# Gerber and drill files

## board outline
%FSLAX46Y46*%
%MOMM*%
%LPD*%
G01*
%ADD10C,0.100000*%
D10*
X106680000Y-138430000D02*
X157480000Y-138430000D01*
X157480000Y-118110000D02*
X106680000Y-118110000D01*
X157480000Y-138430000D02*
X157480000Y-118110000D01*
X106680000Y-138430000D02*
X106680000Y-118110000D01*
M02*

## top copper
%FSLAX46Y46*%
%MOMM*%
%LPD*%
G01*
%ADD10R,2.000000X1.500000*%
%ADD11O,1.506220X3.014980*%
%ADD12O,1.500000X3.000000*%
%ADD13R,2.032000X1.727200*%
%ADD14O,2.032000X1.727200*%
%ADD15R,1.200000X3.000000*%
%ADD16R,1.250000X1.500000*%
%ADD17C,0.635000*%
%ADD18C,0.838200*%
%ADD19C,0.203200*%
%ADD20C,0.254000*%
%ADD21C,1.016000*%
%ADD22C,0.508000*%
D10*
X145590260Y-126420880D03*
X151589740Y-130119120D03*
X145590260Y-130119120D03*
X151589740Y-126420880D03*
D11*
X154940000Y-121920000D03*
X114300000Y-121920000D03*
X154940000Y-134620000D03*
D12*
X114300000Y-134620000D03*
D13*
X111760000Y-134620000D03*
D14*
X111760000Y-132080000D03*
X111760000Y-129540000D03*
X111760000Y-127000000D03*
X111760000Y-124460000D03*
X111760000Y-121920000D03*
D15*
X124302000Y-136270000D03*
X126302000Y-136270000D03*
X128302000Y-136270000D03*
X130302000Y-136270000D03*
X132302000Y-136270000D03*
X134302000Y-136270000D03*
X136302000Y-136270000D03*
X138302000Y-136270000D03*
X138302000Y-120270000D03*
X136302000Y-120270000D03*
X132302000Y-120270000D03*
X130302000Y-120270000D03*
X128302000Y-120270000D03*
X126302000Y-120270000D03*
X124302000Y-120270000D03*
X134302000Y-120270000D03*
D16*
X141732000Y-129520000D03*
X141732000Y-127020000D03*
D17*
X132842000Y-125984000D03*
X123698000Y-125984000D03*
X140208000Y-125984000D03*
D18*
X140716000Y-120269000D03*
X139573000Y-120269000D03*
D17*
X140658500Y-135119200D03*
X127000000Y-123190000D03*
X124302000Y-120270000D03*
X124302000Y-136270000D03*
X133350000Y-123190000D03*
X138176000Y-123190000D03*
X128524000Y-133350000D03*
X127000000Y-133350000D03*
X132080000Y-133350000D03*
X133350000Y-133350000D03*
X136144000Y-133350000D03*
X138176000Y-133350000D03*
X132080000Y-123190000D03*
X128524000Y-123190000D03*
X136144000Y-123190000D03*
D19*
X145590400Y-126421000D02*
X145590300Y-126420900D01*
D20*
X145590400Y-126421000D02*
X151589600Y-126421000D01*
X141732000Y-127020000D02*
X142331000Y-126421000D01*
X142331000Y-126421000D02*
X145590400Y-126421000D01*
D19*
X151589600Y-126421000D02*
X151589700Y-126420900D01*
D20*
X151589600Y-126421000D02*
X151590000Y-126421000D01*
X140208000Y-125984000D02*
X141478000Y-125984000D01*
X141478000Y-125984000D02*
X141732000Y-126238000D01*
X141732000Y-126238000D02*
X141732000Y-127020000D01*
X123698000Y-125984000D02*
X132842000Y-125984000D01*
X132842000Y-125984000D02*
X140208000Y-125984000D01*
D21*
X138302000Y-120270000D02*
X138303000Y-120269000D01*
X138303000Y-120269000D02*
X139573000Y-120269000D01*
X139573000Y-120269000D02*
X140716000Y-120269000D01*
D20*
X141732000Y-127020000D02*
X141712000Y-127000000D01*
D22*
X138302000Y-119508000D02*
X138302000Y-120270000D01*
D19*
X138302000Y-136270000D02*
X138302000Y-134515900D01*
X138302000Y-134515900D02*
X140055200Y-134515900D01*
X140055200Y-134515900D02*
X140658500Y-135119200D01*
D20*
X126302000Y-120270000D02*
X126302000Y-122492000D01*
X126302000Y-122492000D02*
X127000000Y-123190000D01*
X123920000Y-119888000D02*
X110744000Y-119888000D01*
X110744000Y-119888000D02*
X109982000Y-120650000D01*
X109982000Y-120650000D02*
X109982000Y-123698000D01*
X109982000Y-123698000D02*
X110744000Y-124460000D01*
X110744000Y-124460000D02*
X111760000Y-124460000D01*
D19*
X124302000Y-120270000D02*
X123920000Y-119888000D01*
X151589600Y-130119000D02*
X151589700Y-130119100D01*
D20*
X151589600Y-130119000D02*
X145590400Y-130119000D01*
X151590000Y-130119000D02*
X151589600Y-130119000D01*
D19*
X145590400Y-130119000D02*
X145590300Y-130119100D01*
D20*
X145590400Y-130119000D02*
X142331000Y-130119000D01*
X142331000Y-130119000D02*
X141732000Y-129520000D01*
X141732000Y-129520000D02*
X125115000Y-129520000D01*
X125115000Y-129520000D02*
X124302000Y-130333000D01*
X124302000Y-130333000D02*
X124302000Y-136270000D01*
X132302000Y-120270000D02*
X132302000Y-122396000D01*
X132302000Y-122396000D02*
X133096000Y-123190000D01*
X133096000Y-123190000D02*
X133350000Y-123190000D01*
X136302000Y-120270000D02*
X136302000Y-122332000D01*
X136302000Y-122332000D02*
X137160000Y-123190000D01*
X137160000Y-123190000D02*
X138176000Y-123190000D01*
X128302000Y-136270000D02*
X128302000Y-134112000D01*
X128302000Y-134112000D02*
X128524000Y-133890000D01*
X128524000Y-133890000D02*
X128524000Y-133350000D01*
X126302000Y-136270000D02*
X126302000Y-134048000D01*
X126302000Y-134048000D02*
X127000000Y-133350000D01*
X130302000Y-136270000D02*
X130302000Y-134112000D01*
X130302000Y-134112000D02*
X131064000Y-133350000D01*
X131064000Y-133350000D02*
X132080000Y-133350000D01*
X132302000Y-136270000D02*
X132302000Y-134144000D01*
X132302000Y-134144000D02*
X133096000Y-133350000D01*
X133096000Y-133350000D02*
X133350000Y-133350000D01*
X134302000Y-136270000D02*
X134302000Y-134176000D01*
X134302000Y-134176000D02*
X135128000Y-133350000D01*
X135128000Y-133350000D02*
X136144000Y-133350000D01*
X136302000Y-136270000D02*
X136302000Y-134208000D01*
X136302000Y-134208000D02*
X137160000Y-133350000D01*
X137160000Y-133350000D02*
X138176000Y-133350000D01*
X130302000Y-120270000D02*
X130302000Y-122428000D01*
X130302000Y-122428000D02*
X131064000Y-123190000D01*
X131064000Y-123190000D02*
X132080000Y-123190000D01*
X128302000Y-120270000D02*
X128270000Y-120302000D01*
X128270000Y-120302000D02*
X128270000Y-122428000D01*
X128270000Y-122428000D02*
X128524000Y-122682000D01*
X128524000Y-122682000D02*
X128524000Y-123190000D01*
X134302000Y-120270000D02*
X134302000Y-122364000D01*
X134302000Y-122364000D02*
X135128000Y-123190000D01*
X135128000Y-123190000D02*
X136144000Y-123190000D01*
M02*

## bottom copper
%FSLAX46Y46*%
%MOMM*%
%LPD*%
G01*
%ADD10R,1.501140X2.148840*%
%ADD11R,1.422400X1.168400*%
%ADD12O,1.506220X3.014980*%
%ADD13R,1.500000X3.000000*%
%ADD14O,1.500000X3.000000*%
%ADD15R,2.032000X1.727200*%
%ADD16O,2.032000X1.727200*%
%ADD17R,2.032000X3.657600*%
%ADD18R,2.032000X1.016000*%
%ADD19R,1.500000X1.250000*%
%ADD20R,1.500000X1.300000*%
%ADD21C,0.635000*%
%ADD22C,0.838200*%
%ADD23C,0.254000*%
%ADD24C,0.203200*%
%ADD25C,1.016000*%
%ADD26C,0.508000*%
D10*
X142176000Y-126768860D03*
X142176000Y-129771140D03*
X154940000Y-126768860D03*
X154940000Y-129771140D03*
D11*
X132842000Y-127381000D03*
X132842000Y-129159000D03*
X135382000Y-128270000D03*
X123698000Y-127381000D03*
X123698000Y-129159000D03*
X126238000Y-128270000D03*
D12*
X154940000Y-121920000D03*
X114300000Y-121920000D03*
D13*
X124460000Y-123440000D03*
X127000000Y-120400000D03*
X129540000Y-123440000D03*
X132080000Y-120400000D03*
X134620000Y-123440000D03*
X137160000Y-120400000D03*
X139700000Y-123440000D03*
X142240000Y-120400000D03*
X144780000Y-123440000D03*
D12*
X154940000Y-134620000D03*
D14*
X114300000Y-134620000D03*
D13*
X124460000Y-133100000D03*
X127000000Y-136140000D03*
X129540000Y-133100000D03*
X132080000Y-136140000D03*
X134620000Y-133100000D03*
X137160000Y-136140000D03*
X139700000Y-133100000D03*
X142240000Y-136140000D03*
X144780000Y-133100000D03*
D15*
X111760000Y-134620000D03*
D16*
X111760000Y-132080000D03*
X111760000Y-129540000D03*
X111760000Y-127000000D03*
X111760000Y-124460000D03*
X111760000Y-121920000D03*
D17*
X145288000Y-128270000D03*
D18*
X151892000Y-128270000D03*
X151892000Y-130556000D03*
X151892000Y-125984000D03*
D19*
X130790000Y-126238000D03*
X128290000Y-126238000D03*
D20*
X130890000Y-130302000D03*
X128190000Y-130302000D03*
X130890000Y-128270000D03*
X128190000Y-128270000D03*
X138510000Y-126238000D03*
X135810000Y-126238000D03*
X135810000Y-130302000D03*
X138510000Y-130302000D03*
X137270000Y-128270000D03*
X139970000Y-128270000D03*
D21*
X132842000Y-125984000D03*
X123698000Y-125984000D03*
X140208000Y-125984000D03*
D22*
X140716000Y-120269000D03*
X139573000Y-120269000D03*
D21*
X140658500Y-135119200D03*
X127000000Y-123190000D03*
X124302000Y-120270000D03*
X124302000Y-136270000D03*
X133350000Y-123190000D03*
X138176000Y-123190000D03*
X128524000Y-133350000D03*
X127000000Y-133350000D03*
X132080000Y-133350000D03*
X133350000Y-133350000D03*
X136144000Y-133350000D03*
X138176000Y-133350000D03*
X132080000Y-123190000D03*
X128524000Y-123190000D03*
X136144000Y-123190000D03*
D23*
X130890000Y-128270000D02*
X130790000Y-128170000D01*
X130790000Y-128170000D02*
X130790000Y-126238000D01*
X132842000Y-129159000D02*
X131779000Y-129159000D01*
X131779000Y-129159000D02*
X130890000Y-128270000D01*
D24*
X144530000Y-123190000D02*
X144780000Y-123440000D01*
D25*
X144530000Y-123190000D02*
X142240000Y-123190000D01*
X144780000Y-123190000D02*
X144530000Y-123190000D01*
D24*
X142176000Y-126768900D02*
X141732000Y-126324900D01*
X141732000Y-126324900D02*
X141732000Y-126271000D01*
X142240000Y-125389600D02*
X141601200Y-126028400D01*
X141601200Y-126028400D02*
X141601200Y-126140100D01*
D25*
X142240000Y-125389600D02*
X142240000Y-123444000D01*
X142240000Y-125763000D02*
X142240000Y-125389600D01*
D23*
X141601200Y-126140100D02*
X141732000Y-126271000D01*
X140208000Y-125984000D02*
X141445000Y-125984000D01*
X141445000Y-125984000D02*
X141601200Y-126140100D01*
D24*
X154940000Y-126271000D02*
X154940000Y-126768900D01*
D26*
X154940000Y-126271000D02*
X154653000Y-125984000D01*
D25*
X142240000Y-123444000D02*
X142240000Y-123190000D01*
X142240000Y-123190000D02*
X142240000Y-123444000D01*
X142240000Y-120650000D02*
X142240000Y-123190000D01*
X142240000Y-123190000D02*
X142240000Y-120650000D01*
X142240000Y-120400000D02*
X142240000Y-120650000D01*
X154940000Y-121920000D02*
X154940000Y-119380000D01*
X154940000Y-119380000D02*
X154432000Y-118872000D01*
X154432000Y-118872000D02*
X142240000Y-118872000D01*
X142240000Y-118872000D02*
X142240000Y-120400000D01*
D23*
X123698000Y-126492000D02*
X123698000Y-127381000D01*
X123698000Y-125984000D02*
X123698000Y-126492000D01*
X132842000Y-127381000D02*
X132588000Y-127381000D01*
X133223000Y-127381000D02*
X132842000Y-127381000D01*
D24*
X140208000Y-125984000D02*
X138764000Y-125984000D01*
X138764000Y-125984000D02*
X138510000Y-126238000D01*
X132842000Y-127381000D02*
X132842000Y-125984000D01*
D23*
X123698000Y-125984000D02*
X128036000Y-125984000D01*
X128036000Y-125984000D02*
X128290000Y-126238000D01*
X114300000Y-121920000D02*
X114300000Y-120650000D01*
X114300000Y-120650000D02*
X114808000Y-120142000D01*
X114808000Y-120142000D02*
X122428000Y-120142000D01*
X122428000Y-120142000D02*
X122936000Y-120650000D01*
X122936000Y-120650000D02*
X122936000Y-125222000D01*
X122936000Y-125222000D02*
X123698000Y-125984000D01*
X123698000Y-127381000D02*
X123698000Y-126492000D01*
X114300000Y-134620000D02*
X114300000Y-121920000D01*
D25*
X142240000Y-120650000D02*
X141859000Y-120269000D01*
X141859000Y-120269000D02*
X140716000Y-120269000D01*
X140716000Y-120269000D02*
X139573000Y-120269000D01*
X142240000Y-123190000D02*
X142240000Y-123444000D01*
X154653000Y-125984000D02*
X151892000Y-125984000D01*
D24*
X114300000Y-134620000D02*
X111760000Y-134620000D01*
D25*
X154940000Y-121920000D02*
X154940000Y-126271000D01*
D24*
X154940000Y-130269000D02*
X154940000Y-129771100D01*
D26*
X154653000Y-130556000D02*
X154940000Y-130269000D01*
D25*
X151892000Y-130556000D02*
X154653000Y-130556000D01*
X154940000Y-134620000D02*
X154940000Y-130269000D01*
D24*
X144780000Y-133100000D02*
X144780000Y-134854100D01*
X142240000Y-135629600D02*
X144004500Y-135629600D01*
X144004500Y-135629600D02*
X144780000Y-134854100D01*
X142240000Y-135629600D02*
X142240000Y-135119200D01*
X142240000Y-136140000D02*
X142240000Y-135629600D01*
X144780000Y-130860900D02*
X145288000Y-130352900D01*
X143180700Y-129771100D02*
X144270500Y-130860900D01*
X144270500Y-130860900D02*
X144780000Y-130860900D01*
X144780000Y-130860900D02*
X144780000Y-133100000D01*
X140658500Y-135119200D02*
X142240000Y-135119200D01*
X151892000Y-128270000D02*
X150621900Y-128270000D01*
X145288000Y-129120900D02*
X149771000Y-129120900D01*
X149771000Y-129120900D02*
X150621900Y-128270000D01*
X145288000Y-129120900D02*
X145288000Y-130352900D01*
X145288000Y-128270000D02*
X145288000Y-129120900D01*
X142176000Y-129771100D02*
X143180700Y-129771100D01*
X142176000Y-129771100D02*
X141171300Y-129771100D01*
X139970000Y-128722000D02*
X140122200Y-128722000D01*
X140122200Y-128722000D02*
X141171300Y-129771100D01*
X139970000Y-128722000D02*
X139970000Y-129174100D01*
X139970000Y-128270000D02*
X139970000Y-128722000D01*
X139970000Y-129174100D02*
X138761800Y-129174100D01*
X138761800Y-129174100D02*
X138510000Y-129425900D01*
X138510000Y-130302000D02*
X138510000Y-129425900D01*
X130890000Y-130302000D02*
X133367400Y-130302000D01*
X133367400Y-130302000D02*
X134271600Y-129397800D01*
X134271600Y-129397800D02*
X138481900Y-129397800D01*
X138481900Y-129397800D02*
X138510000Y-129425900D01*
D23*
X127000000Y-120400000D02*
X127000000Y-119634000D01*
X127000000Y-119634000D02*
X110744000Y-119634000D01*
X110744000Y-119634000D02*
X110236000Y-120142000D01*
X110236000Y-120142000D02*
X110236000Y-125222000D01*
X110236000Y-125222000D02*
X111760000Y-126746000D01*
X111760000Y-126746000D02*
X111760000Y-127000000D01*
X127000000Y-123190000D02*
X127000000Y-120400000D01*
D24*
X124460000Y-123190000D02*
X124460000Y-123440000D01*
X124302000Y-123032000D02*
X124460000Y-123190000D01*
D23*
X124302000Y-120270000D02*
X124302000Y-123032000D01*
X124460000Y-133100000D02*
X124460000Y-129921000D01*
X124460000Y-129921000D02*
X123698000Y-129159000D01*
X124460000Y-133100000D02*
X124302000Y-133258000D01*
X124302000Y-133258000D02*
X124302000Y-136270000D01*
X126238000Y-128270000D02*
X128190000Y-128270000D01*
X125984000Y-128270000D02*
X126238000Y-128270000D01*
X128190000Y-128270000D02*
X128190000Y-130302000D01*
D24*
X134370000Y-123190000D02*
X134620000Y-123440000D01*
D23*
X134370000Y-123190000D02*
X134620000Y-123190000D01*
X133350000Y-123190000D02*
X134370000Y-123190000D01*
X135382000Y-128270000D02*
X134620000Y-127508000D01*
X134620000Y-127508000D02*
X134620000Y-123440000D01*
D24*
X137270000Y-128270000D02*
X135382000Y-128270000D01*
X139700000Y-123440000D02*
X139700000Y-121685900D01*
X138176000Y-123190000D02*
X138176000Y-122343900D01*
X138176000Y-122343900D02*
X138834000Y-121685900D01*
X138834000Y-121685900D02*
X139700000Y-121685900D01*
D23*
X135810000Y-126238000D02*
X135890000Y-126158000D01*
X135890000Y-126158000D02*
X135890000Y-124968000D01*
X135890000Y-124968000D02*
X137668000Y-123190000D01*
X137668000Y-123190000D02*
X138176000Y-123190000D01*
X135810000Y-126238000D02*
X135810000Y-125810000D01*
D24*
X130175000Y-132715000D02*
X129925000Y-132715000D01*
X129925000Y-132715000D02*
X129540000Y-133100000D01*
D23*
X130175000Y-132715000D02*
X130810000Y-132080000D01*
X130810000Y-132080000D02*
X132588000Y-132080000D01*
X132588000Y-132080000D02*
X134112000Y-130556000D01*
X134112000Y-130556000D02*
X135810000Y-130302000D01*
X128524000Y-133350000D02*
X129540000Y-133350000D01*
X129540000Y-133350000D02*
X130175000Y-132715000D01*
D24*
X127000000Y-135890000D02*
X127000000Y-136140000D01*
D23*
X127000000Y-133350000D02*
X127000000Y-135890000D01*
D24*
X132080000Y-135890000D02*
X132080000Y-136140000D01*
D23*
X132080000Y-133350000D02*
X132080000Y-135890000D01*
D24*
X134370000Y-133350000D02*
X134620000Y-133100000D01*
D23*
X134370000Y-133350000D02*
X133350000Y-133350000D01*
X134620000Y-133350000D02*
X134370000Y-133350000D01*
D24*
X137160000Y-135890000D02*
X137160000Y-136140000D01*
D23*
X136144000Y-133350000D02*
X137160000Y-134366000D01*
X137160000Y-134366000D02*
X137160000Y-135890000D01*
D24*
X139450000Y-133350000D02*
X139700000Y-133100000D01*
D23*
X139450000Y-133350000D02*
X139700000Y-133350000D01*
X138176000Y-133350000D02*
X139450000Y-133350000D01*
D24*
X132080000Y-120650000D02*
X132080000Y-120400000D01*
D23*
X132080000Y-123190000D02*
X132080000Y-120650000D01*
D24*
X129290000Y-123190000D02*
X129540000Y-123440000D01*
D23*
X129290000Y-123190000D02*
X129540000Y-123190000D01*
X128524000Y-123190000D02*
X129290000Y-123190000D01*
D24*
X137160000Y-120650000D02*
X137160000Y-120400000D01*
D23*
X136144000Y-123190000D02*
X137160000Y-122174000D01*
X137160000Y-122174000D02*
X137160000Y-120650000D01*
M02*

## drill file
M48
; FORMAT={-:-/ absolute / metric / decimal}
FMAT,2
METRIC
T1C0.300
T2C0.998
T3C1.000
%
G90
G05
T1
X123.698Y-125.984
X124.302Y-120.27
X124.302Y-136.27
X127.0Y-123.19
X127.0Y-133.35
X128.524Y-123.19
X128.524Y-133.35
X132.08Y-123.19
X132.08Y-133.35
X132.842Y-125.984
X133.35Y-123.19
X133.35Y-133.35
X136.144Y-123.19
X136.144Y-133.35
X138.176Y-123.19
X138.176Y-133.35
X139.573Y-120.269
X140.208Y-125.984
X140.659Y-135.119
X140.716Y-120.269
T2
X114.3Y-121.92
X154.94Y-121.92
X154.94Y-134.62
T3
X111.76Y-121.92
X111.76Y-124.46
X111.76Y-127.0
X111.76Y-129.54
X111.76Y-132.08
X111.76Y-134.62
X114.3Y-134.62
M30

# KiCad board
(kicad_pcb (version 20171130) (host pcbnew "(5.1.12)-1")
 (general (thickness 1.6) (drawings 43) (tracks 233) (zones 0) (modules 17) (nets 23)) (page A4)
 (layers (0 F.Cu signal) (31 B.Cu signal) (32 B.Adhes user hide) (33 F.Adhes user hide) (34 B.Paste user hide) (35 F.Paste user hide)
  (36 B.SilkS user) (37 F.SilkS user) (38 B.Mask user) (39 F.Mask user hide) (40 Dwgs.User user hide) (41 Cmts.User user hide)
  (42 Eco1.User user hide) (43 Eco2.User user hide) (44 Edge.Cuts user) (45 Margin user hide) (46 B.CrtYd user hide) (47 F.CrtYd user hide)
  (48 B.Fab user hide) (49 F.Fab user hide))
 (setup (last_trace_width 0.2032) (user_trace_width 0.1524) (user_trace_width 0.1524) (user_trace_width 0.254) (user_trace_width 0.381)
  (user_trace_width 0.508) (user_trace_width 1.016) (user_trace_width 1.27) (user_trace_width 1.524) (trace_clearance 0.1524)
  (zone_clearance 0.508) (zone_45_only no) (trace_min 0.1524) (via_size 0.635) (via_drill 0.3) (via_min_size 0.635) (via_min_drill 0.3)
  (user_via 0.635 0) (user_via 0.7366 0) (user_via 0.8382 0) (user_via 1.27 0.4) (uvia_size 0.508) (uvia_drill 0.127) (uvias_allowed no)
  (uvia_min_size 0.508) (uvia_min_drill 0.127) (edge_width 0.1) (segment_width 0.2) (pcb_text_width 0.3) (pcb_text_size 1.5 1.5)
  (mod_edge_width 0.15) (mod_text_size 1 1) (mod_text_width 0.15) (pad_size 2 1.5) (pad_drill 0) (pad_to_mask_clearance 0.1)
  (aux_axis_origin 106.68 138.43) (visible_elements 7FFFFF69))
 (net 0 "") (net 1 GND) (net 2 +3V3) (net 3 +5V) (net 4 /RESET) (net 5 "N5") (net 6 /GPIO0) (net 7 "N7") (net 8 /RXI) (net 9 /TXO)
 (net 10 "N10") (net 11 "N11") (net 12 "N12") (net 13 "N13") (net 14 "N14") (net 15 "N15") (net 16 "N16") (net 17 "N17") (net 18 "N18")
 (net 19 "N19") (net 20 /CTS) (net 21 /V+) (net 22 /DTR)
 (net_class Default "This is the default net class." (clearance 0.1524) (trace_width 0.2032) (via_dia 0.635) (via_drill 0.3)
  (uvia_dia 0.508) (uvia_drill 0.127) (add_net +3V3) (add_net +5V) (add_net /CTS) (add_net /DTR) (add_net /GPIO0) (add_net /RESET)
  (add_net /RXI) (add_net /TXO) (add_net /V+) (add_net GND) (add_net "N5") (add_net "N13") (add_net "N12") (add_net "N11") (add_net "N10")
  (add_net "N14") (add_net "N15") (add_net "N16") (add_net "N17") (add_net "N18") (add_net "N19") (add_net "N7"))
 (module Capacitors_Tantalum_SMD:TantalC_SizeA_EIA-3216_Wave (layer B.Cu) (at 142.176 128.27 90)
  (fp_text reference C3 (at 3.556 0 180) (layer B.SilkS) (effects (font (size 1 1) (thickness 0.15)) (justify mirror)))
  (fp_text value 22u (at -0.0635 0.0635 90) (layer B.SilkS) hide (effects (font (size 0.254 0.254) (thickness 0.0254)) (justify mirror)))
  (pad 2 smd rect (at 1.50114 0 90) (size 2.14884 1.50114) (layers B.Cu B.Paste B.Mask) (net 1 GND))
  (pad 1 smd rect (at -1.50114 0 90) (size 2.14884 1.50114) (layers B.Cu B.Paste B.Mask) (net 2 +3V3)))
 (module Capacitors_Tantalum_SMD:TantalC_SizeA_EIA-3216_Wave (layer B.Cu) (at 154.94 128.27 90)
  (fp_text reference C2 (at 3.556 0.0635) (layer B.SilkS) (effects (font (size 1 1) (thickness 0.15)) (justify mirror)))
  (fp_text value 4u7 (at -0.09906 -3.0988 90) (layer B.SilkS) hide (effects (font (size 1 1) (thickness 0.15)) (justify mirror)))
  (pad 2 smd rect (at 1.50114 0 90) (size 2.14884 1.50114) (layers B.Cu B.Paste B.Mask) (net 1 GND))
  (pad 1 smd rect (at -1.50114 0 90) (size 2.14884 1.50114) (layers B.Cu B.Paste B.Mask) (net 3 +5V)))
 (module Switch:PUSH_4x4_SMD (layer F.Cu) (at 148.59 128.27) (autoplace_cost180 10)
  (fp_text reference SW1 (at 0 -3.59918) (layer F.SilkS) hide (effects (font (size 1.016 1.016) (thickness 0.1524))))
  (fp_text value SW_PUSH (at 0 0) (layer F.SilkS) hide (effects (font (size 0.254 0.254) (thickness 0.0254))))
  (pad 1 smd rect (at -2.99974 -1.84912) (size 2 1.5) (layers F.Cu F.Paste F.Mask) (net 1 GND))
  (pad 2 smd rect (at 2.99974 1.84912) (size 2 1.5) (layers F.Cu F.Paste F.Mask) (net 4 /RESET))
  (pad 2 smd rect (at -2.99974 1.84912) (size 2 1.5) (layers F.Cu F.Paste F.Mask) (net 4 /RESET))
  (pad 1 smd rect (at 2.99974 -1.84912) (size 2 1.5) (layers F.Cu F.Paste F.Mask) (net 1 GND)))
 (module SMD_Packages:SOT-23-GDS (layer B.Cu) (at 134.112 128.27 270)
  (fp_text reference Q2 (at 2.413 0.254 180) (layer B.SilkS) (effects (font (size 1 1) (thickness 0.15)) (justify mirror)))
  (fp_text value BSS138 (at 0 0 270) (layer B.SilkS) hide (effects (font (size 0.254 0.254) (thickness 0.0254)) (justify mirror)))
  (pad S smd rect (at -0.889 1.27 270) (size 1.1684 1.4224) (layers B.Cu B.Paste B.Mask) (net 1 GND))
  (pad G smd rect (at 0.889 1.27 270) (size 1.1684 1.4224) (layers B.Cu B.Paste B.Mask) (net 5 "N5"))
  (pad D smd rect (at 0 -1.27 270) (size 1.1684 1.4224) (layers B.Cu B.Paste B.Mask) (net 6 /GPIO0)))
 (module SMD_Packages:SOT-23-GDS (layer B.Cu) (at 124.968 128.27 270)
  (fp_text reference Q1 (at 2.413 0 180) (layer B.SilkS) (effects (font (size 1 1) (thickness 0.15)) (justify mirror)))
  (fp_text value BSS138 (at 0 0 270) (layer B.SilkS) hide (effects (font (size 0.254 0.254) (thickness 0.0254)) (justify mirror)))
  (pad S smd rect (at -0.889 1.27 270) (size 1.1684 1.4224) (layers B.Cu B.Paste B.Mask) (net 1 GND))
  (pad G smd rect (at 0.889 1.27 270) (size 1.1684 1.4224) (layers B.Cu B.Paste B.Mask) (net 4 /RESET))
  (pad D smd rect (at 0 -1.27 270) (size 1.1684 1.4224) (layers B.Cu B.Paste B.Mask) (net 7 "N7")))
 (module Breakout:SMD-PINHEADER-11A (layer B.Cu) (at 114.3 121.92)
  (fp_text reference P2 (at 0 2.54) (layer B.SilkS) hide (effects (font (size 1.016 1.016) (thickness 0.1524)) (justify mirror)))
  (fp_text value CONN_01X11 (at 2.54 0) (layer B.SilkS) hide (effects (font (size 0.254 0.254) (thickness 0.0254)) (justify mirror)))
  (pad 11 thru_hole oval (at 40.64 0) (size 1.50622 3.01498) (drill 0.99822) (layers *.Cu *.Mask) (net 1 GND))
  (pad 1 thru_hole oval (at 0 0) (size 1.50622 3.01498) (drill 0.99822) (layers *.Cu *.Mask) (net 1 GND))
  (pad 2 smd rect (at 10.16 1.52) (size 1.5 3) (layers B.Cu B.Paste B.Mask) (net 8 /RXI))
  (pad 3 smd rect (at 12.7 -1.52) (size 1.5 3) (layers B.Cu B.Paste B.Mask) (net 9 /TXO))
  (pad 4 smd rect (at 15.24 1.52) (size 1.5 3) (layers B.Cu B.Paste B.Mask) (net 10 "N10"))
  (pad 5 smd rect (at 17.78 -1.52) (size 1.5 3) (layers B.Cu B.Paste B.Mask) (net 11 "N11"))
  (pad 6 smd rect (at 20.32 1.52) (size 1.5 3) (layers B.Cu B.Paste B.Mask) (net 6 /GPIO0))
  (pad 7 smd rect (at 22.86 -1.52) (size 1.5 3) (layers B.Cu B.Paste B.Mask) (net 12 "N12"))
  (pad 8 smd rect (at 25.4 1.52) (size 1.5 3) (layers B.Cu B.Paste B.Mask) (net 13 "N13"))
  (pad 9 smd rect (at 27.94 -1.52) (size 1.5 3) (layers B.Cu B.Paste B.Mask) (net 1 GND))
  (pad 10 smd rect (at 30.48 1.52) (size 1.5 3) (layers B.Cu B.Paste B.Mask) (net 1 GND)))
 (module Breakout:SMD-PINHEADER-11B (layer B.Cu) (at 114.3 134.62)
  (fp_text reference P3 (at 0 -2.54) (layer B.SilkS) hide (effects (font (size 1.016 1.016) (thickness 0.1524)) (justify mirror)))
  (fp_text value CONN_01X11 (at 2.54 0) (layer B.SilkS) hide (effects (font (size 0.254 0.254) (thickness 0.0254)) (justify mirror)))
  (pad 11 thru_hole oval (at 40.64 0) (size 1.50622 3.01498) (drill 0.99822) (layers *.Cu *.Mask) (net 3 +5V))
  (pad 1 thru_hole oval (at 0 0) (size 1.5 3) (drill 1) (layers *.Cu *.Mask) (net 1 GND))
  (pad 2 smd rect (at 10.16 -1.52) (size 1.5 3) (layers B.Cu B.Paste B.Mask) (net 4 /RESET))
  (pad 3 smd rect (at 12.7 1.52) (size 1.5 3) (layers B.Cu B.Paste B.Mask) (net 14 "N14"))
  (pad 4 smd rect (at 15.24 -1.52) (size 1.5 3) (layers B.Cu B.Paste B.Mask) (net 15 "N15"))
  (pad 5 smd rect (at 17.78 1.52) (size 1.5 3) (layers B.Cu B.Paste B.Mask) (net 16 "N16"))
  (pad 6 smd rect (at 20.32 -1.52) (size 1.5 3) (layers B.Cu B.Paste B.Mask) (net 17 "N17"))
  (pad 7 smd rect (at 22.86 1.52) (size 1.5 3) (layers B.Cu B.Paste B.Mask) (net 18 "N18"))
  (pad 8 smd rect (at 25.4 -1.52) (size 1.5 3) (layers B.Cu B.Paste B.Mask) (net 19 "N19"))
  (pad 9 smd rect (at 27.94 1.52) (size 1.5 3) (layers B.Cu B.Paste B.Mask) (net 2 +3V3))
  (pad 10 smd rect (at 30.48 -1.52) (size 1.5 3) (layers B.Cu B.Paste B.Mask) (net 2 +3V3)))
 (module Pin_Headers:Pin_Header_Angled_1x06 (layer F.Cu) (at 111.76 128.27 90)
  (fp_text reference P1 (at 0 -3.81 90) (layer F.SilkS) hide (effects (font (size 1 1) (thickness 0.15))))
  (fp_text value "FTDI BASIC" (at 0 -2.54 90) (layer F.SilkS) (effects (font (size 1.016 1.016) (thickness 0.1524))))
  (pad 1 thru_hole rect (at -6.35 0 90) (size 1.7272 2.032) (drill 1) (layers *.Cu *.Mask F.SilkS) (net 1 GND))
  (pad 2 thru_hole oval (at -3.81 0 90) (size 1.7272 2.032) (drill 1) (layers *.Cu *.Mask F.SilkS) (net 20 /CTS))
  (pad 3 thru_hole oval (at -1.27 0 90) (size 1.7272 2.032) (drill 1) (layers *.Cu *.Mask F.SilkS) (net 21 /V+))
  (pad 4 thru_hole oval (at 1.27 0 90) (size 1.7272 2.032) (drill 1) (layers *.Cu *.Mask F.SilkS) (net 9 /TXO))
  (pad 5 thru_hole oval (at 3.81 0 90) (size 1.7272 2.032) (drill 1) (layers *.Cu *.Mask F.SilkS) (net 8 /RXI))
  (pad 6 thru_hole oval (at 6.35 0 90) (size 1.7272 2.032) (drill 1) (layers *.Cu *.Mask F.SilkS) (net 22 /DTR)))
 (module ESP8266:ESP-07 (layer F.Cu) (at 130.302 128.27)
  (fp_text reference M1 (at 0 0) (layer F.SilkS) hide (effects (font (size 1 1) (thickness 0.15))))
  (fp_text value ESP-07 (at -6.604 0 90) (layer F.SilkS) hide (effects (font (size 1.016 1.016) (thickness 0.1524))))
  (pad 1 smd rect (at -6 8) (size 1.2 3) (layers F.Cu F.Paste F.Mask) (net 4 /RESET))
  (pad 2 smd rect (at -4 8) (size 1.2 3) (layers F.Cu F.Paste F.Mask) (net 14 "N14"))
  (pad 3 smd rect (at -2 8) (size 1.2 3) (layers F.Cu F.Paste F.Mask) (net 15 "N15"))
  (pad 4 smd rect (at 0 8) (size 1.2 3) (layers F.Cu F.Paste F.Mask) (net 16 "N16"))
  (pad 5 smd rect (at 2 8) (size 1.2 3) (layers F.Cu F.Paste F.Mask) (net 17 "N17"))
  (pad 6 smd rect (at 4 8) (size 1.2 3) (layers F.Cu F.Paste F.Mask) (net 18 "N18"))
  (pad 7 smd rect (at 6 8) (size 1.2 3) (layers F.Cu F.Paste F.Mask) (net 19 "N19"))
  (pad 8 smd rect (at 8 8) (size 1.2 3) (layers F.Cu F.Paste F.Mask) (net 2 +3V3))
  (pad 9 smd rect (at 8 -8) (size 1.2 3) (layers F.Cu F.Paste F.Mask) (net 1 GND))
  (pad 10 smd rect (at 6 -8) (size 1.2 3) (layers F.Cu F.Paste F.Mask) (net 13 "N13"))
  (pad 12 smd rect (at 2 -8) (size 1.2 3) (layers F.Cu F.Paste F.Mask) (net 6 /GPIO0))
  (pad 13 smd rect (at 0 -8) (size 1.2 3) (layers F.Cu F.Paste F.Mask) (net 11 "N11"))
  (pad 14 smd rect (at -2 -8) (size 1.2 3) (layers F.Cu F.Paste F.Mask) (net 10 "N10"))
  (pad 15 smd rect (at -4 -8) (size 1.2 3) (layers F.Cu F.Paste F.Mask) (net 9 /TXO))
  (pad 16 smd rect (at -6 -8) (size 1.2 3) (layers F.Cu F.Paste F.Mask) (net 8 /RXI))
  (pad 11 smd rect (at 4 -8) (size 1.2 3) (layers F.Cu F.Paste F.Mask) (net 12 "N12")))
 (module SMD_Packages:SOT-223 (layer B.Cu) (at 148.59 128.27 270)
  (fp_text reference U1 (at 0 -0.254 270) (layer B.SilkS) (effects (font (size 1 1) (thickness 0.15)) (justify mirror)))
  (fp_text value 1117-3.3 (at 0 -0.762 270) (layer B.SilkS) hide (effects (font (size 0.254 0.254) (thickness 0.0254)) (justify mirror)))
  (pad 2 smd rect (at 0 3.302 270) (size 3.6576 2.032) (layers B.Cu B.Paste B.Mask) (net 2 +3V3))
  (pad 2 smd rect (at 0 -3.302 270) (size 1.016 2.032) (layers B.Cu B.Paste B.Mask) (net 2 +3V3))
  (pad 3 smd rect (at 2.286 -3.302 270) (size 1.016 2.032) (layers B.Cu B.Paste B.Mask) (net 3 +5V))
  (pad 1 smd rect (at -2.286 -3.302 270) (size 1.016 2.032) (layers B.Cu B.Paste B.Mask) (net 1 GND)))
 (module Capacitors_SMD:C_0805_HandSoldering (layer B.Cu) (at 129.54 126.238 180)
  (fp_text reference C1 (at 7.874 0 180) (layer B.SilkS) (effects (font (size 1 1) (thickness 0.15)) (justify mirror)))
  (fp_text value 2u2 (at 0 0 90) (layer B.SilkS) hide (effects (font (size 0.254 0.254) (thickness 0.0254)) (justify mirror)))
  (pad 1 smd rect (at -1.25 0 180) (size 1.5 1.25) (layers B.Cu B.Paste B.Mask) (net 5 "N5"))
  (pad 2 smd rect (at 1.25 0 180) (size 1.5 1.25) (layers B.Cu B.Paste B.Mask) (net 1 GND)))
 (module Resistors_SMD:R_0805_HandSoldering (layer B.Cu) (at 129.54 130.302 180)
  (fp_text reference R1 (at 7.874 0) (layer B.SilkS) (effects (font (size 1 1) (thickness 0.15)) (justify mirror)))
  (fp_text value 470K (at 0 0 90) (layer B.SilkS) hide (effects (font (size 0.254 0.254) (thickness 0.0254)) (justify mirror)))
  (pad 1 smd rect (at -1.35 0 180) (size 1.5 1.3) (layers B.Cu B.Paste B.Mask) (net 2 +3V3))
  (pad 2 smd rect (at 1.35 0 180) (size 1.5 1.3) (layers B.Cu B.Paste B.Mask) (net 7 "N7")))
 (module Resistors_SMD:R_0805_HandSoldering (layer B.Cu) (at 129.54 128.27 180)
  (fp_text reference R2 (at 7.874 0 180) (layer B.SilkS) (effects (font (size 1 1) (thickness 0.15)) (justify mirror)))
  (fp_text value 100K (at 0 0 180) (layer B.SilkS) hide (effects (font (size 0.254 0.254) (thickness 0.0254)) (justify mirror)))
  (pad 1 smd rect (at -1.35 0 180) (size 1.5 1.3) (layers B.Cu B.Paste B.Mask) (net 5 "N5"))
  (pad 2 smd rect (at 1.35 0 180) (size 1.5 1.3) (layers B.Cu B.Paste B.Mask) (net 7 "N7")))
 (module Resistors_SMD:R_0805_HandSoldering (layer B.Cu) (at 137.16 126.238 180)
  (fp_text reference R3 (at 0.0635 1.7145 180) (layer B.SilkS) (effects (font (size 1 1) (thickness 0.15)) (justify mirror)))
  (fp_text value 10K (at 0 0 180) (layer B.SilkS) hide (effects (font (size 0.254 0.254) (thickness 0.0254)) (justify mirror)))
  (pad 1 smd rect (at -1.35 0 180) (size 1.5 1.3) (layers B.Cu B.Paste B.Mask) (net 1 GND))
  (pad 2 smd rect (at 1.35 0 180) (size 1.5 1.3) (layers B.Cu B.Paste B.Mask) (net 13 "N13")))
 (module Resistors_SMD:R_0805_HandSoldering (layer B.Cu) (at 137.16 130.302)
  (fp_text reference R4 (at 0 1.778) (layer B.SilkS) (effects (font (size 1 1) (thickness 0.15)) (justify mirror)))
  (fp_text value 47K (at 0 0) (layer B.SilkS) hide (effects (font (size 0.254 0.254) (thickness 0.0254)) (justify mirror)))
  (pad 1 smd rect (at -1.35 0) (size 1.5 1.3) (layers B.Cu B.Paste B.Mask) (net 15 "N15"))
  (pad 2 smd rect (at 1.35 0) (size 1.5 1.3) (layers B.Cu B.Paste B.Mask) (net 2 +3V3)))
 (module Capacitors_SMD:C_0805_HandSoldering (layer F.Cu) (at 141.732 128.27 90)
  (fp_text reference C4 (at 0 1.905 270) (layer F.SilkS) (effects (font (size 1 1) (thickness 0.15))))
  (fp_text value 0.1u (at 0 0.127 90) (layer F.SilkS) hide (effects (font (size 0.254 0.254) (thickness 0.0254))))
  (pad 1 smd rect (at -1.25 0 90) (size 1.5 1.25) (layers F.Cu F.Paste F.Mask) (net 4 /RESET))
  (pad 2 smd rect (at 1.25 0 90) (size 1.5 1.25) (layers F.Cu F.Paste F.Mask) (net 1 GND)))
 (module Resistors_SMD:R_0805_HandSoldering (layer B.Cu) (at 138.62 128.27)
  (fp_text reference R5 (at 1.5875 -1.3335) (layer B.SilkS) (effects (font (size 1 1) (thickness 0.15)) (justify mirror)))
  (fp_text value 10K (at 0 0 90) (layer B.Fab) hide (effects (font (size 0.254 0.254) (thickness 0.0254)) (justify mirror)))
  (pad 1 smd rect (at -1.35 0) (size 1.5 1.3) (layers B.Cu B.Paste B.Mask) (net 6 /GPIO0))
  (pad 2 smd rect (at 1.35 0) (size 1.5 1.3) (layers B.Cu B.Paste B.Mask) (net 2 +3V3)))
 (gr_line (start 106.68 138.43) (end 157.48 138.43) (angle 90) (layer Edge.Cuts) (width 0.1))
 (gr_line (start 157.48 118.11) (end 106.68 118.11) (angle 90) (layer Edge.Cuts) (width 0.1))
 (gr_line (start 157.48 138.43) (end 157.48 118.11) (angle 90) (layer Edge.Cuts) (width 0.1))
 (gr_line (start 106.68 138.43) (end 106.68 118.11) (angle 90) (layer Edge.Cuts) (width 0.1))
 (segment (start 130.89 128.27) (end 130.79 128.17) (width 0.254) (layer B.Cu) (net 5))
 (segment (start 130.79 128.17) (end 130.79 126.238) (width 0.254) (layer B.Cu) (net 5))
 (segment (start 132.842 129.159) (end 131.779 129.159) (width 0.254) (layer B.Cu) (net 5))
 (segment (start 131.779 129.159) (end 130.89 128.27) (width 0.254) (layer B.Cu) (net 5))
 (segment (start 144.53 123.19) (end 144.78 123.44) (width 0.2032) (layer B.Cu) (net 1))
 (segment (start 144.53 123.19) (end 142.24 123.19) (width 1.016) (layer B.Cu) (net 1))
 (segment (start 144.78 123.19) (end 144.53 123.19) (width 1.016) (layer B.Cu) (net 1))
 (segment (start 142.176 126.7689) (end 141.732 126.3249) (width 0.2032) (layer B.Cu) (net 1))
 (segment (start 141.732 126.3249) (end 141.732 126.271) (width 0.2032) (layer B.Cu) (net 1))
 (segment (start 142.24 125.3896) (end 141.6012 126.0284) (width 0.2032) (layer B.Cu) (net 1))
 (segment (start 141.6012 126.0284) (end 141.6012 126.1401) (width 0.2032) (layer B.Cu) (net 1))
 (segment (start 142.24 125.3896) (end 142.24 123.444) (width 1.016) (layer B.Cu) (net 1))
 (segment (start 142.24 125.763) (end 142.24 125.3896) (width 1.016) (layer B.Cu) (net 1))
 (segment (start 141.6012 126.1401) (end 141.732 126.271) (width 0.254) (layer B.Cu) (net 1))
 (segment (start 140.208 125.984) (end 141.445 125.984) (width 0.254) (layer B.Cu) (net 1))
 (segment (start 141.445 125.984) (end 141.6012 126.1401) (width 0.254) (layer B.Cu) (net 1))
 (segment (start 145.5904 126.421) (end 145.5903 126.4209) (width 0.2032) (layer F.Cu) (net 1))
 (segment (start 145.5904 126.421) (end 151.5896 126.421) (width 0.254) (layer F.Cu) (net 1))
 (segment (start 141.732 127.02) (end 142.331 126.421) (width 0.254) (layer F.Cu) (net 1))
 (segment (start 142.331 126.421) (end 145.5904 126.421) (width 0.254) (layer F.Cu) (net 1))
 (segment (start 154.94 126.271) (end 154.94 126.7689) (width 0.2032) (layer B.Cu) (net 1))
 (segment (start 154.94 126.271) (end 154.653 125.984) (width 0.508) (layer B.Cu) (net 1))
 (segment (start 151.5896 126.421) (end 151.5897 126.4209) (width 0.2032) (layer F.Cu) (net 1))
 (segment (start 151.5896 126.421) (end 151.59 126.421) (width 0.254) (layer F.Cu) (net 1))
 (segment (start 142.24 123.444) (end 142.24 123.19) (width 1.016) (layer B.Cu) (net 1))
 (segment (start 142.24 123.19) (end 142.24 123.444) (width 1.016) (layer B.Cu) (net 1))
 (segment (start 142.24 120.65) (end 142.24 123.19) (width 1.016) (layer B.Cu) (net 1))
 (segment (start 142.24 123.19) (end 142.24 120.65) (width 1.016) (layer B.Cu) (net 1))
 (segment (start 142.24 120.4) (end 142.24 120.65) (width 1.016) (layer B.Cu) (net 1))
 (segment (start 154.94 121.92) (end 154.94 119.38) (width 1.016) (layer B.Cu) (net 1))
 (segment (start 154.94 119.38) (end 154.432 118.872) (width 1.016) (layer B.Cu) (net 1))
 (segment (start 154.432 118.872) (end 142.24 118.872) (width 1.016) (layer B.Cu) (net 1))
 (segment (start 142.24 118.872) (end 142.24 120.4) (width 1.016) (layer B.Cu) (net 1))
 (segment (start 123.698 126.492) (end 123.698 127.381) (width 0.254) (layer B.Cu) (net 1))
 (segment (start 123.698 125.984) (end 123.698 126.492) (width 0.254) (layer B.Cu) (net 1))
 (segment (start 132.842 127.381) (end 132.588 127.381) (width 0.254) (layer B.Cu) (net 1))
 (segment (start 133.223 127.381) (end 132.842 127.381) (width 0.254) (layer B.Cu) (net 1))
 (segment (start 140.208 125.984) (end 138.764 125.984) (width 0.2032) (layer B.Cu) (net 1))
 (segment (start 138.764 125.984) (end 138.51 126.238) (width 0.2032) (layer B.Cu) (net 1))
 (segment (start 132.842 127.381) (end 132.842 125.984) (width 0.2032) (layer B.Cu) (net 1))
 (segment (start 140.208 125.984) (end 141.478 125.984) (width 0.254) (layer F.Cu) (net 1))
 (segment (start 141.478 125.984) (end 141.732 126.238) (width 0.254) (layer F.Cu) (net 1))
 (segment (start 141.732 126.238) (end 141.732 127.02) (width 0.254) (layer F.Cu) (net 1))
 (segment (start 123.698 125.984) (end 132.842 125.984) (width 0.254) (layer F.Cu) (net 1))
 (segment (start 132.842 125.984) (end 140.208 125.984) (width 0.254) (layer F.Cu) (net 1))
 (segment (start 123.698 125.984) (end 128.036 125.984) (width 0.254) (layer B.Cu) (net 1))
 (segment (start 128.036 125.984) (end 128.29 126.238) (width 0.254) (layer B.Cu) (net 1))
 (segment (start 114.3 121.92) (end 114.3 120.65) (width 0.254) (layer B.Cu) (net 1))
 (segment (start 114.3 120.65) (end 114.808 120.142) (width 0.254) (layer B.Cu) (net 1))
 (segment (start 114.808 120.142) (end 122.428 120.142) (width 0.254) (layer B.Cu) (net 1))
 (segment (start 122.428 120.142) (end 122.936 120.65) (width 0.254) (layer B.Cu) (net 1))
 (segment (start 122.936 120.65) (end 122.936 125.222) (width 0.254) (layer B.Cu) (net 1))
 (segment (start 122.936 125.222) (end 123.698 125.984) (width 0.254) (layer B.Cu) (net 1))
 (segment (start 123.698 127.381) (end 123.698 126.492) (width 0.254) (layer B.Cu) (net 1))
 (segment (start 114.3 134.62) (end 114.3 121.92) (width 0.254) (layer B.Cu) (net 1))
 (segment (start 142.24 120.65) (end 141.859 120.269) (width 1.016) (layer B.Cu) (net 1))
 (segment (start 141.859 120.269) (end 140.716 120.269) (width 1.016) (layer B.Cu) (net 1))
 (segment (start 140.716 120.269) (end 139.573 120.269) (width 1.016) (layer B.Cu) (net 1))
 (segment (start 138.302 120.27) (end 138.303 120.269) (width 1.016) (layer F.Cu) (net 1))
 (segment (start 138.303 120.269) (end 139.573 120.269) (width 1.016) (layer F.Cu) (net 1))
 (segment (start 139.573 120.269) (end 140.716 120.269) (width 1.016) (layer F.Cu) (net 1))
 (segment (start 141.732 127.02) (end 141.712 127) (width 0.254) (layer F.Cu) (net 1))
 (segment (start 142.24 123.19) (end 142.24 123.444) (width 1.016) (layer B.Cu) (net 1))
 (segment (start 138.302 119.508) (end 138.302 120.27) (width 0.508) (layer F.Cu) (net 1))
 (segment (start 154.653 125.984) (end 151.892 125.984) (width 1.016) (layer B.Cu) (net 1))
 (segment (start 114.3 134.62) (end 111.76 134.62) (width 0.2032) (layer B.Cu) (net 1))
 (segment (start 154.94 121.92) (end 154.94 126.271) (width 1.016) (layer B.Cu) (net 1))
 (via (at 132.842 125.984) (size 0.635) (layers F.Cu B.Cu) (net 1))
 (via (at 123.698 125.984) (size 0.635) (layers F.Cu B.Cu) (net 1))
 (via (at 140.208 125.984) (size 0.635) (layers F.Cu B.Cu) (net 1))
 (via (at 140.716 120.269) (size 0.8382) (layers F.Cu B.Cu) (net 1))
 (via (at 139.573 120.269) (size 0.8382) (layers F.Cu B.Cu) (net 1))
 (segment (start 154.94 130.269) (end 154.94 129.7711) (width 0.2032) (layer B.Cu) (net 3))
 (segment (start 154.653 130.556) (end 154.94 130.269) (width 0.508) (layer B.Cu) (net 3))
 (segment (start 151.892 130.556) (end 154.653 130.556) (width 1.016) (layer B.Cu) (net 3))
 (segment (start 154.94 134.62) (end 154.94 130.269) (width 1.016) (layer B.Cu) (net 3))
 (segment (start 144.78 133.1) (end 144.78 134.8541) (width 0.2032) (layer B.Cu) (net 2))
 (segment (start 142.24 135.6296) (end 144.0045 135.6296) (width 0.2032) (layer B.Cu) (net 2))
 (segment (start 144.0045 135.6296) (end 144.78 134.8541) (width 0.2032) (layer B.Cu) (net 2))
 (segment (start 142.24 135.6296) (end 142.24 135.1192) (width 0.2032) (layer B.Cu) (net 2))
 (segment (start 142.24 136.14) (end 142.24 135.6296) (width 0.2032) (layer B.Cu) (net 2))
 (segment (start 144.78 130.8609) (end 145.288 130.3529) (width 0.2032) (layer B.Cu) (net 2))
 (segment (start 143.1807 129.7711) (end 144.2705 130.8609) (width 0.2032) (layer B.Cu) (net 2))
 (segment (start 144.2705 130.8609) (end 144.78 130.8609) (width 0.2032) (layer B.Cu) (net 2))
 (segment (start 144.78 130.8609) (end 144.78 133.1) (width 0.2032) (layer B.Cu) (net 2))
 (segment (start 138.302 136.27) (end 138.302 134.5159) (width 0.2032) (layer F.Cu) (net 2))
 (segment (start 140.6585 135.1192) (end 142.24 135.1192) (width 0.2032) (layer B.Cu) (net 2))
 (segment (start 138.302 134.5159) (end 140.0552 134.5159) (width 0.2032) (layer F.Cu) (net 2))
 (segment (start 140.0552 134.5159) (end 140.6585 135.1192) (width 0.2032) (layer F.Cu) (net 2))
 (segment (start 151.892 128.27) (end 150.6219 128.27) (width 0.2032) (layer B.Cu) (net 2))
 (segment (start 145.288 129.1209) (end 149.771 129.1209) (width 0.2032) (layer B.Cu) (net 2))
 (segment (start 149.771 129.1209) (end 150.6219 128.27) (width 0.2032) (layer B.Cu) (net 2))
 (segment (start 145.288 129.1209) (end 145.288 130.3529) (width 0.2032) (layer B.Cu) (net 2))
 (segment (start 145.288 128.27) (end 145.288 129.1209) (width 0.2032) (layer B.Cu) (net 2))
 (segment (start 142.176 129.7711) (end 143.1807 129.7711) (width 0.2032) (layer B.Cu) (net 2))
 (segment (start 142.176 129.7711) (end 141.1713 129.7711) (width 0.2032) (layer B.Cu) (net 2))
 (segment (start 139.97 128.722) (end 140.1222 128.722) (width 0.2032) (layer B.Cu) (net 2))
 (segment (start 140.1222 128.722) (end 141.1713 129.7711) (width 0.2032) (layer B.Cu) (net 2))
 (segment (start 139.97 128.722) (end 139.97 129.1741) (width 0.2032) (layer B.Cu) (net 2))
 (segment (start 139.97 128.27) (end 139.97 128.722) (width 0.2032) (layer B.Cu) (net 2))
 (segment (start 139.97 129.1741) (end 138.7618 129.1741) (width 0.2032) (layer B.Cu) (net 2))
 (segment (start 138.7618 129.1741) (end 138.51 129.4259) (width 0.2032) (layer B.Cu) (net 2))
 (segment (start 138.51 130.302) (end 138.51 129.4259) (width 0.2032) (layer B.Cu) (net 2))
 (segment (start 130.89 130.302) (end 133.3674 130.302) (width 0.2032) (layer B.Cu) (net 2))
 (segment (start 133.3674 130.302) (end 134.2716 129.3978) (width 0.2032) (layer B.Cu) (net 2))
 (segment (start 134.2716 129.3978) (end 138.4819 129.3978) (width 0.2032) (layer B.Cu) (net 2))
 (segment (start 138.4819 129.3978) (end 138.51 129.4259) (width 0.2032) (layer B.Cu) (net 2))
 (via (at 140.6585 135.1192) (size 0.635) (layers F.Cu B.Cu) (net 2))
 (segment (start 127 120.4) (end 127 119.634) (width 0.254) (layer B.Cu) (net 9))
 (segment (start 127 119.634) (end 110.744 119.634) (width 0.254) (layer B.Cu) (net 9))
 (segment (start 110.744 119.634) (end 110.236 120.142) (width 0.254) (layer B.Cu) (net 9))
 (segment (start 110.236 120.142) (end 110.236 125.222) (width 0.254) (layer B.Cu) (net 9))
 (segment (start 110.236 125.222) (end 111.76 126.746) (width 0.254) (layer B.Cu) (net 9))
 (segment (start 111.76 126.746) (end 111.76 127) (width 0.254) (layer B.Cu) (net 9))
 (segment (start 127 123.19) (end 127 120.4) (width 0.254) (layer B.Cu) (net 9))
 (segment (start 126.302 120.27) (end 126.302 122.492) (width 0.254) (layer F.Cu) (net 9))
 (segment (start 126.302 122.492) (end 127 123.19) (width 0.254) (layer F.Cu) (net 9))
 (via (at 127 123.19) (size 0.635) (layers F.Cu B.Cu) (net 9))
 (segment (start 124.46 123.19) (end 124.46 123.44) (width 0.2032) (layer B.Cu) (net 8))
 (segment (start 124.302 123.032) (end 124.46 123.19) (width 0.2032) (layer B.Cu) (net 8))
 (segment (start 123.92 119.888) (end 110.744 119.888) (width 0.254) (layer F.Cu) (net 8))
 (segment (start 110.744 119.888) (end 109.982 120.65) (width 0.254) (layer F.Cu) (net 8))
 (segment (start 109.982 120.65) (end 109.982 123.698) (width 0.254) (layer F.Cu) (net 8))
 (segment (start 109.982 123.698) (end 110.744 124.46) (width 0.254) (layer F.Cu) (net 8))
 (segment (start 110.744 124.46) (end 111.76 124.46) (width 0.254) (layer F.Cu) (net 8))
 (segment (start 124.302 120.27) (end 123.92 119.888) (width 0.2032) (layer F.Cu) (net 8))
 (segment (start 124.302 120.27) (end 124.302 123.032) (width 0.254) (layer B.Cu) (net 8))
 (via (at 124.302 120.27) (size 0.635) (layers F.Cu B.Cu) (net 8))
 (segment (start 151.5896 130.119) (end 151.5897 130.1191) (width 0.2032) (layer F.Cu) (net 4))
 (segment (start 151.5896 130.119) (end 145.5904 130.119) (width 0.254) (layer F.Cu) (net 4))
 (segment (start 151.59 130.119) (end 151.5896 130.119) (width 0.254) (layer F.Cu) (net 4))
 (segment (start 145.5904 130.119) (end 145.5903 130.1191) (width 0.2032) (layer F.Cu) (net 4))
 (segment (start 145.5904 130.119) (end 142.331 130.119) (width 0.254) (layer F.Cu) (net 4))
 (segment (start 142.331 130.119) (end 141.732 129.52) (width 0.254) (layer F.Cu) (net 4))
 (segment (start 124.46 133.1) (end 124.46 129.921) (width 0.254) (layer B.Cu) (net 4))
 (segment (start 124.46 129.921) (end 123.698 129.159) (width 0.254) (layer B.Cu) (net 4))
 (segment (start 124.46 133.1) (end 124.302 133.258) (width 0.254) (layer B.Cu) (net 4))
 (segment (start 124.302 133.258) (end 124.302 136.27) (width 0.254) (layer B.Cu) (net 4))
 (segment (start 141.732 129.52) (end 125.115 129.52) (width 0.254) (layer F.Cu) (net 4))
 (segment (start 125.115 129.52) (end 124.302 130.333) (width 0.254) (layer F.Cu) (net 4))
 (segment (start 124.302 130.333) (end 124.302 136.27) (width 0.254) (layer F.Cu) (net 4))
 (via (at 124.302 136.27) (size 0.635) (layers F.Cu B.Cu) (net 4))
 (segment (start 126.238 128.27) (end 128.19 128.27) (width 0.254) (layer B.Cu) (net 7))
 (segment (start 125.984 128.27) (end 126.238 128.27) (width 0.254) (layer B.Cu) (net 7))
 (segment (start 128.19 128.27) (end 128.19 130.302) (width 0.254) (layer B.Cu) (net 7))
 (segment (start 134.37 123.19) (end 134.62 123.44) (width 0.2032) (layer B.Cu) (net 6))
 (segment (start 134.37 123.19) (end 134.62 123.19) (width 0.254) (layer B.Cu) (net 6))
 (segment (start 133.35 123.19) (end 134.37 123.19) (width 0.254) (layer B.Cu) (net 6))
 (segment (start 135.382 128.27) (end 134.62 127.508) (width 0.254) (layer B.Cu) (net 6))
 (segment (start 134.62 127.508) (end 134.62 123.44) (width 0.254) (layer B.Cu) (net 6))
 (segment (start 132.302 120.27) (end 132.302 122.396) (width 0.254) (layer F.Cu) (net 6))
 (segment (start 132.302 122.396) (end 133.096 123.19) (width 0.254) (layer F.Cu) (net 6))
 (segment (start 133.096 123.19) (end 133.35 123.19) (width 0.254) (layer F.Cu) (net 6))
 (segment (start 137.27 128.27) (end 135.382 128.27) (width 0.2032) (layer B.Cu) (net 6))
 (via (at 133.35 123.19) (size 0.635) (layers F.Cu B.Cu) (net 6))
 (segment (start 139.7 123.44) (end 139.7 121.6859) (width 0.2032) (layer B.Cu) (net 13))
 (segment (start 138.176 123.19) (end 138.176 122.3439) (width 0.2032) (layer B.Cu) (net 13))
 (segment (start 138.176 122.3439) (end 138.834 121.6859) (width 0.2032) (layer B.Cu) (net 13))
 (segment (start 138.834 121.6859) (end 139.7 121.6859) (width 0.2032) (layer B.Cu) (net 13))
 (segment (start 136.302 120.27) (end 136.302 122.332) (width 0.254) (layer F.Cu) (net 13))
 (segment (start 136.302 122.332) (end 137.16 123.19) (width 0.254) (layer F.Cu) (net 13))
 (segment (start 137.16 123.19) (end 138.176 123.19) (width 0.254) (layer F.Cu) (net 13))
 (segment (start 135.81 126.238) (end 135.89 126.158) (width 0.254) (layer B.Cu) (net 13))
 (segment (start 135.89 126.158) (end 135.89 124.968) (width 0.254) (layer B.Cu) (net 13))
 (segment (start 135.89 124.968) (end 137.668 123.19) (width 0.254) (layer B.Cu) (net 13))
 (segment (start 137.668 123.19) (end 138.176 123.19) (width 0.254) (layer B.Cu) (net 13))
 (segment (start 135.81 126.238) (end 135.81 125.81) (width 0.254) (layer B.Cu) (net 13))
 (via (at 138.176 123.19) (size 0.635) (layers F.Cu B.Cu) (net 13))
 (segment (start 130.175 132.715) (end 129.925 132.715) (width 0.2032) (layer B.Cu) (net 15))
 (segment (start 129.925 132.715) (end 129.54 133.1) (width 0.2032) (layer B.Cu) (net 15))
 (segment (start 130.175 132.715) (end 130.81 132.08) (width 0.254) (layer B.Cu) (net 15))
 (segment (start 130.81 132.08) (end 132.588 132.08) (width 0.254) (layer B.Cu) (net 15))
 (segment (start 132.588 132.08) (end 134.112 130.556) (width 0.254) (layer B.Cu) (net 15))
 (segment (start 134.112 130.556) (end 135.81 130.302) (width 0.254) (layer B.Cu) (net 15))
 (segment (start 128.524 133.35) (end 129.54 133.35) (width 0.254) (layer B.Cu) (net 15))
 (segment (start 129.54 133.35) (end 130.175 132.715) (width 0.254) (layer B.Cu) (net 15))
 (segment (start 128.302 136.27) (end 128.302 134.112) (width 0.254) (layer F.Cu) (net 15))
 (segment (start 128.302 134.112) (end 128.524 133.89) (width 0.254) (layer F.Cu) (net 15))
 (segment (start 128.524 133.89) (end 128.524 133.35) (width 0.254) (layer F.Cu) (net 15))
 (via (at 128.524 133.35) (size 0.635) (layers F.Cu B.Cu) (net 15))
 (segment (start 127 135.89) (end 127 136.14) (width 0.2032) (layer B.Cu) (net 14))
 (segment (start 127 133.35) (end 127 135.89) (width 0.254) (layer B.Cu) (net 14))
 (segment (start 126.302 136.27) (end 126.302 134.048) (width 0.254) (layer F.Cu) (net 14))
 (segment (start 126.302 134.048) (end 127 133.35) (width 0.254) (layer F.Cu) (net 14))
 (via (at 127 133.35) (size 0.635) (layers F.Cu B.Cu) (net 14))
 (segment (start 132.08 135.89) (end 132.08 136.14) (width 0.2032) (layer B.Cu) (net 16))
 (segment (start 132.08 133.35) (end 132.08 135.89) (width 0.254) (layer B.Cu) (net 16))
 (segment (start 130.302 136.27) (end 130.302 134.112) (width 0.254) (layer F.Cu) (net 16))
 (segment (start 130.302 134.112) (end 131.064 133.35) (width 0.254) (layer F.Cu) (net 16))
 (segment (start 131.064 133.35) (end 132.08 133.35) (width 0.254) (layer F.Cu) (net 16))
 (via (at 132.08 133.35) (size 0.635) (layers F.Cu B.Cu) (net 16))
 (segment (start 134.37 133.35) (end 134.62 133.1) (width 0.2032) (layer B.Cu) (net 17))
 (segment (start 134.37 133.35) (end 133.35 133.35) (width 0.254) (layer B.Cu) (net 17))
 (segment (start 134.62 133.35) (end 134.37 133.35) (width 0.254) (layer B.Cu) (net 17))
 (segment (start 132.302 136.27) (end 132.302 134.144) (width 0.254) (layer F.Cu) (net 17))
 (segment (start 132.302 134.144) (end 133.096 133.35) (width 0.254) (layer F.Cu) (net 17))
 (segment (start 133.096 133.35) (end 133.35 133.35) (width 0.254) (layer F.Cu) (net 17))
 (via (at 133.35 133.35) (size 0.635) (layers F.Cu B.Cu) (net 17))
 (segment (start 137.16 135.89) (end 137.16 136.14) (width 0.2032) (layer B.Cu) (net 18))
 (segment (start 136.144 133.35) (end 137.16 134.366) (width 0.254) (layer B.Cu) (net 18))
 (segment (start 137.16 134.366) (end 137.16 135.89) (width 0.254) (layer B.Cu) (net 18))
 (segment (start 134.302 136.27) (end 134.302 134.176) (width 0.254) (layer F.Cu) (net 18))
 (segment (start 134.302 134.176) (end 135.128 133.35) (width 0.254) (layer F.Cu) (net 18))
 (segment (start 135.128 133.35) (end 136.144 133.35) (width 0.254) (layer F.Cu) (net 18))
 (via (at 136.144 133.35) (size 0.635) (layers F.Cu B.Cu) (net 18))
 (segment (start 139.45 133.35) (end 139.7 133.1) (width 0.2032) (layer B.Cu) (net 19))
 (segment (start 139.45 133.35) (end 139.7 133.35) (width 0.254) (layer B.Cu) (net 19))
 (segment (start 138.176 133.35) (end 139.45 133.35) (width 0.254) (layer B.Cu) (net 19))
 (segment (start 136.302 136.27) (end 136.302 134.208) (width 0.254) (layer F.Cu) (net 19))
 (segment (start 136.302 134.208) (end 137.16 133.35) (width 0.254) (layer F.Cu) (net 19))
 (segment (start 137.16 133.35) (end 138.176 133.35) (width 0.254) (layer F.Cu) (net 19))
 (via (at 138.176 133.35) (size 0.635) (layers F.Cu B.Cu) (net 19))
 (segment (start 132.08 120.65) (end 132.08 120.4) (width 0.2032) (layer B.Cu) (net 11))
 (segment (start 132.08 123.19) (end 132.08 120.65) (width 0.254) (layer B.Cu) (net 11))
 (segment (start 130.302 120.27) (end 130.302 122.428) (width 0.254) (layer F.Cu) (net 11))
 (segment (start 130.302 122.428) (end 131.064 123.19) (width 0.254) (layer F.Cu) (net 11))
 (segment (start 131.064 123.19) (end 132.08 123.19) (width 0.254) (layer F.Cu) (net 11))
 (via (at 132.08 123.19) (size 0.635) (layers F.Cu B.Cu) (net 11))
 (segment (start 129.29 123.19) (end 129.54 123.44) (width 0.2032) (layer B.Cu) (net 10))
 (segment (start 129.29 123.19) (end 129.54 123.19) (width 0.254) (layer B.Cu) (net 10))
 (segment (start 128.524 123.19) (end 129.29 123.19) (width 0.254) (layer B.Cu) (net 10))
 (segment (start 128.302 120.27) (end 128.27 120.302) (width 0.254) (layer F.Cu) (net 10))
 (segment (start 128.27 120.302) (end 128.27 122.428) (width 0.254) (layer F.Cu) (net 10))
 (segment (start 128.27 122.428) (end 128.524 122.682) (width 0.254) (layer F.Cu) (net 10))
 (segment (start 128.524 122.682) (end 128.524 123.19) (width 0.254) (layer F.Cu) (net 10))
 (via (at 128.524 123.19) (size 0.635) (layers F.Cu B.Cu) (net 10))
 (segment (start 137.16 120.65) (end 137.16 120.4) (width 0.2032) (layer B.Cu) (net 12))
 (segment (start 136.144 123.19) (end 137.16 122.174) (width 0.254) (layer B.Cu) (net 12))
 (segment (start 137.16 122.174) (end 137.16 120.65) (width 0.254) (layer B.Cu) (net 12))
 (segment (start 134.302 120.27) (end 134.302 122.364) (width 0.254) (layer F.Cu) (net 12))
 (segment (start 134.302 122.364) (end 135.128 123.19) (width 0.254) (layer F.Cu) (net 12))
 (segment (start 135.128 123.19) (end 136.144 123.19) (width 0.254) (layer F.Cu) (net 12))
 (via (at 136.144 123.19) (size 0.635) (layers F.Cu B.Cu) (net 12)))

